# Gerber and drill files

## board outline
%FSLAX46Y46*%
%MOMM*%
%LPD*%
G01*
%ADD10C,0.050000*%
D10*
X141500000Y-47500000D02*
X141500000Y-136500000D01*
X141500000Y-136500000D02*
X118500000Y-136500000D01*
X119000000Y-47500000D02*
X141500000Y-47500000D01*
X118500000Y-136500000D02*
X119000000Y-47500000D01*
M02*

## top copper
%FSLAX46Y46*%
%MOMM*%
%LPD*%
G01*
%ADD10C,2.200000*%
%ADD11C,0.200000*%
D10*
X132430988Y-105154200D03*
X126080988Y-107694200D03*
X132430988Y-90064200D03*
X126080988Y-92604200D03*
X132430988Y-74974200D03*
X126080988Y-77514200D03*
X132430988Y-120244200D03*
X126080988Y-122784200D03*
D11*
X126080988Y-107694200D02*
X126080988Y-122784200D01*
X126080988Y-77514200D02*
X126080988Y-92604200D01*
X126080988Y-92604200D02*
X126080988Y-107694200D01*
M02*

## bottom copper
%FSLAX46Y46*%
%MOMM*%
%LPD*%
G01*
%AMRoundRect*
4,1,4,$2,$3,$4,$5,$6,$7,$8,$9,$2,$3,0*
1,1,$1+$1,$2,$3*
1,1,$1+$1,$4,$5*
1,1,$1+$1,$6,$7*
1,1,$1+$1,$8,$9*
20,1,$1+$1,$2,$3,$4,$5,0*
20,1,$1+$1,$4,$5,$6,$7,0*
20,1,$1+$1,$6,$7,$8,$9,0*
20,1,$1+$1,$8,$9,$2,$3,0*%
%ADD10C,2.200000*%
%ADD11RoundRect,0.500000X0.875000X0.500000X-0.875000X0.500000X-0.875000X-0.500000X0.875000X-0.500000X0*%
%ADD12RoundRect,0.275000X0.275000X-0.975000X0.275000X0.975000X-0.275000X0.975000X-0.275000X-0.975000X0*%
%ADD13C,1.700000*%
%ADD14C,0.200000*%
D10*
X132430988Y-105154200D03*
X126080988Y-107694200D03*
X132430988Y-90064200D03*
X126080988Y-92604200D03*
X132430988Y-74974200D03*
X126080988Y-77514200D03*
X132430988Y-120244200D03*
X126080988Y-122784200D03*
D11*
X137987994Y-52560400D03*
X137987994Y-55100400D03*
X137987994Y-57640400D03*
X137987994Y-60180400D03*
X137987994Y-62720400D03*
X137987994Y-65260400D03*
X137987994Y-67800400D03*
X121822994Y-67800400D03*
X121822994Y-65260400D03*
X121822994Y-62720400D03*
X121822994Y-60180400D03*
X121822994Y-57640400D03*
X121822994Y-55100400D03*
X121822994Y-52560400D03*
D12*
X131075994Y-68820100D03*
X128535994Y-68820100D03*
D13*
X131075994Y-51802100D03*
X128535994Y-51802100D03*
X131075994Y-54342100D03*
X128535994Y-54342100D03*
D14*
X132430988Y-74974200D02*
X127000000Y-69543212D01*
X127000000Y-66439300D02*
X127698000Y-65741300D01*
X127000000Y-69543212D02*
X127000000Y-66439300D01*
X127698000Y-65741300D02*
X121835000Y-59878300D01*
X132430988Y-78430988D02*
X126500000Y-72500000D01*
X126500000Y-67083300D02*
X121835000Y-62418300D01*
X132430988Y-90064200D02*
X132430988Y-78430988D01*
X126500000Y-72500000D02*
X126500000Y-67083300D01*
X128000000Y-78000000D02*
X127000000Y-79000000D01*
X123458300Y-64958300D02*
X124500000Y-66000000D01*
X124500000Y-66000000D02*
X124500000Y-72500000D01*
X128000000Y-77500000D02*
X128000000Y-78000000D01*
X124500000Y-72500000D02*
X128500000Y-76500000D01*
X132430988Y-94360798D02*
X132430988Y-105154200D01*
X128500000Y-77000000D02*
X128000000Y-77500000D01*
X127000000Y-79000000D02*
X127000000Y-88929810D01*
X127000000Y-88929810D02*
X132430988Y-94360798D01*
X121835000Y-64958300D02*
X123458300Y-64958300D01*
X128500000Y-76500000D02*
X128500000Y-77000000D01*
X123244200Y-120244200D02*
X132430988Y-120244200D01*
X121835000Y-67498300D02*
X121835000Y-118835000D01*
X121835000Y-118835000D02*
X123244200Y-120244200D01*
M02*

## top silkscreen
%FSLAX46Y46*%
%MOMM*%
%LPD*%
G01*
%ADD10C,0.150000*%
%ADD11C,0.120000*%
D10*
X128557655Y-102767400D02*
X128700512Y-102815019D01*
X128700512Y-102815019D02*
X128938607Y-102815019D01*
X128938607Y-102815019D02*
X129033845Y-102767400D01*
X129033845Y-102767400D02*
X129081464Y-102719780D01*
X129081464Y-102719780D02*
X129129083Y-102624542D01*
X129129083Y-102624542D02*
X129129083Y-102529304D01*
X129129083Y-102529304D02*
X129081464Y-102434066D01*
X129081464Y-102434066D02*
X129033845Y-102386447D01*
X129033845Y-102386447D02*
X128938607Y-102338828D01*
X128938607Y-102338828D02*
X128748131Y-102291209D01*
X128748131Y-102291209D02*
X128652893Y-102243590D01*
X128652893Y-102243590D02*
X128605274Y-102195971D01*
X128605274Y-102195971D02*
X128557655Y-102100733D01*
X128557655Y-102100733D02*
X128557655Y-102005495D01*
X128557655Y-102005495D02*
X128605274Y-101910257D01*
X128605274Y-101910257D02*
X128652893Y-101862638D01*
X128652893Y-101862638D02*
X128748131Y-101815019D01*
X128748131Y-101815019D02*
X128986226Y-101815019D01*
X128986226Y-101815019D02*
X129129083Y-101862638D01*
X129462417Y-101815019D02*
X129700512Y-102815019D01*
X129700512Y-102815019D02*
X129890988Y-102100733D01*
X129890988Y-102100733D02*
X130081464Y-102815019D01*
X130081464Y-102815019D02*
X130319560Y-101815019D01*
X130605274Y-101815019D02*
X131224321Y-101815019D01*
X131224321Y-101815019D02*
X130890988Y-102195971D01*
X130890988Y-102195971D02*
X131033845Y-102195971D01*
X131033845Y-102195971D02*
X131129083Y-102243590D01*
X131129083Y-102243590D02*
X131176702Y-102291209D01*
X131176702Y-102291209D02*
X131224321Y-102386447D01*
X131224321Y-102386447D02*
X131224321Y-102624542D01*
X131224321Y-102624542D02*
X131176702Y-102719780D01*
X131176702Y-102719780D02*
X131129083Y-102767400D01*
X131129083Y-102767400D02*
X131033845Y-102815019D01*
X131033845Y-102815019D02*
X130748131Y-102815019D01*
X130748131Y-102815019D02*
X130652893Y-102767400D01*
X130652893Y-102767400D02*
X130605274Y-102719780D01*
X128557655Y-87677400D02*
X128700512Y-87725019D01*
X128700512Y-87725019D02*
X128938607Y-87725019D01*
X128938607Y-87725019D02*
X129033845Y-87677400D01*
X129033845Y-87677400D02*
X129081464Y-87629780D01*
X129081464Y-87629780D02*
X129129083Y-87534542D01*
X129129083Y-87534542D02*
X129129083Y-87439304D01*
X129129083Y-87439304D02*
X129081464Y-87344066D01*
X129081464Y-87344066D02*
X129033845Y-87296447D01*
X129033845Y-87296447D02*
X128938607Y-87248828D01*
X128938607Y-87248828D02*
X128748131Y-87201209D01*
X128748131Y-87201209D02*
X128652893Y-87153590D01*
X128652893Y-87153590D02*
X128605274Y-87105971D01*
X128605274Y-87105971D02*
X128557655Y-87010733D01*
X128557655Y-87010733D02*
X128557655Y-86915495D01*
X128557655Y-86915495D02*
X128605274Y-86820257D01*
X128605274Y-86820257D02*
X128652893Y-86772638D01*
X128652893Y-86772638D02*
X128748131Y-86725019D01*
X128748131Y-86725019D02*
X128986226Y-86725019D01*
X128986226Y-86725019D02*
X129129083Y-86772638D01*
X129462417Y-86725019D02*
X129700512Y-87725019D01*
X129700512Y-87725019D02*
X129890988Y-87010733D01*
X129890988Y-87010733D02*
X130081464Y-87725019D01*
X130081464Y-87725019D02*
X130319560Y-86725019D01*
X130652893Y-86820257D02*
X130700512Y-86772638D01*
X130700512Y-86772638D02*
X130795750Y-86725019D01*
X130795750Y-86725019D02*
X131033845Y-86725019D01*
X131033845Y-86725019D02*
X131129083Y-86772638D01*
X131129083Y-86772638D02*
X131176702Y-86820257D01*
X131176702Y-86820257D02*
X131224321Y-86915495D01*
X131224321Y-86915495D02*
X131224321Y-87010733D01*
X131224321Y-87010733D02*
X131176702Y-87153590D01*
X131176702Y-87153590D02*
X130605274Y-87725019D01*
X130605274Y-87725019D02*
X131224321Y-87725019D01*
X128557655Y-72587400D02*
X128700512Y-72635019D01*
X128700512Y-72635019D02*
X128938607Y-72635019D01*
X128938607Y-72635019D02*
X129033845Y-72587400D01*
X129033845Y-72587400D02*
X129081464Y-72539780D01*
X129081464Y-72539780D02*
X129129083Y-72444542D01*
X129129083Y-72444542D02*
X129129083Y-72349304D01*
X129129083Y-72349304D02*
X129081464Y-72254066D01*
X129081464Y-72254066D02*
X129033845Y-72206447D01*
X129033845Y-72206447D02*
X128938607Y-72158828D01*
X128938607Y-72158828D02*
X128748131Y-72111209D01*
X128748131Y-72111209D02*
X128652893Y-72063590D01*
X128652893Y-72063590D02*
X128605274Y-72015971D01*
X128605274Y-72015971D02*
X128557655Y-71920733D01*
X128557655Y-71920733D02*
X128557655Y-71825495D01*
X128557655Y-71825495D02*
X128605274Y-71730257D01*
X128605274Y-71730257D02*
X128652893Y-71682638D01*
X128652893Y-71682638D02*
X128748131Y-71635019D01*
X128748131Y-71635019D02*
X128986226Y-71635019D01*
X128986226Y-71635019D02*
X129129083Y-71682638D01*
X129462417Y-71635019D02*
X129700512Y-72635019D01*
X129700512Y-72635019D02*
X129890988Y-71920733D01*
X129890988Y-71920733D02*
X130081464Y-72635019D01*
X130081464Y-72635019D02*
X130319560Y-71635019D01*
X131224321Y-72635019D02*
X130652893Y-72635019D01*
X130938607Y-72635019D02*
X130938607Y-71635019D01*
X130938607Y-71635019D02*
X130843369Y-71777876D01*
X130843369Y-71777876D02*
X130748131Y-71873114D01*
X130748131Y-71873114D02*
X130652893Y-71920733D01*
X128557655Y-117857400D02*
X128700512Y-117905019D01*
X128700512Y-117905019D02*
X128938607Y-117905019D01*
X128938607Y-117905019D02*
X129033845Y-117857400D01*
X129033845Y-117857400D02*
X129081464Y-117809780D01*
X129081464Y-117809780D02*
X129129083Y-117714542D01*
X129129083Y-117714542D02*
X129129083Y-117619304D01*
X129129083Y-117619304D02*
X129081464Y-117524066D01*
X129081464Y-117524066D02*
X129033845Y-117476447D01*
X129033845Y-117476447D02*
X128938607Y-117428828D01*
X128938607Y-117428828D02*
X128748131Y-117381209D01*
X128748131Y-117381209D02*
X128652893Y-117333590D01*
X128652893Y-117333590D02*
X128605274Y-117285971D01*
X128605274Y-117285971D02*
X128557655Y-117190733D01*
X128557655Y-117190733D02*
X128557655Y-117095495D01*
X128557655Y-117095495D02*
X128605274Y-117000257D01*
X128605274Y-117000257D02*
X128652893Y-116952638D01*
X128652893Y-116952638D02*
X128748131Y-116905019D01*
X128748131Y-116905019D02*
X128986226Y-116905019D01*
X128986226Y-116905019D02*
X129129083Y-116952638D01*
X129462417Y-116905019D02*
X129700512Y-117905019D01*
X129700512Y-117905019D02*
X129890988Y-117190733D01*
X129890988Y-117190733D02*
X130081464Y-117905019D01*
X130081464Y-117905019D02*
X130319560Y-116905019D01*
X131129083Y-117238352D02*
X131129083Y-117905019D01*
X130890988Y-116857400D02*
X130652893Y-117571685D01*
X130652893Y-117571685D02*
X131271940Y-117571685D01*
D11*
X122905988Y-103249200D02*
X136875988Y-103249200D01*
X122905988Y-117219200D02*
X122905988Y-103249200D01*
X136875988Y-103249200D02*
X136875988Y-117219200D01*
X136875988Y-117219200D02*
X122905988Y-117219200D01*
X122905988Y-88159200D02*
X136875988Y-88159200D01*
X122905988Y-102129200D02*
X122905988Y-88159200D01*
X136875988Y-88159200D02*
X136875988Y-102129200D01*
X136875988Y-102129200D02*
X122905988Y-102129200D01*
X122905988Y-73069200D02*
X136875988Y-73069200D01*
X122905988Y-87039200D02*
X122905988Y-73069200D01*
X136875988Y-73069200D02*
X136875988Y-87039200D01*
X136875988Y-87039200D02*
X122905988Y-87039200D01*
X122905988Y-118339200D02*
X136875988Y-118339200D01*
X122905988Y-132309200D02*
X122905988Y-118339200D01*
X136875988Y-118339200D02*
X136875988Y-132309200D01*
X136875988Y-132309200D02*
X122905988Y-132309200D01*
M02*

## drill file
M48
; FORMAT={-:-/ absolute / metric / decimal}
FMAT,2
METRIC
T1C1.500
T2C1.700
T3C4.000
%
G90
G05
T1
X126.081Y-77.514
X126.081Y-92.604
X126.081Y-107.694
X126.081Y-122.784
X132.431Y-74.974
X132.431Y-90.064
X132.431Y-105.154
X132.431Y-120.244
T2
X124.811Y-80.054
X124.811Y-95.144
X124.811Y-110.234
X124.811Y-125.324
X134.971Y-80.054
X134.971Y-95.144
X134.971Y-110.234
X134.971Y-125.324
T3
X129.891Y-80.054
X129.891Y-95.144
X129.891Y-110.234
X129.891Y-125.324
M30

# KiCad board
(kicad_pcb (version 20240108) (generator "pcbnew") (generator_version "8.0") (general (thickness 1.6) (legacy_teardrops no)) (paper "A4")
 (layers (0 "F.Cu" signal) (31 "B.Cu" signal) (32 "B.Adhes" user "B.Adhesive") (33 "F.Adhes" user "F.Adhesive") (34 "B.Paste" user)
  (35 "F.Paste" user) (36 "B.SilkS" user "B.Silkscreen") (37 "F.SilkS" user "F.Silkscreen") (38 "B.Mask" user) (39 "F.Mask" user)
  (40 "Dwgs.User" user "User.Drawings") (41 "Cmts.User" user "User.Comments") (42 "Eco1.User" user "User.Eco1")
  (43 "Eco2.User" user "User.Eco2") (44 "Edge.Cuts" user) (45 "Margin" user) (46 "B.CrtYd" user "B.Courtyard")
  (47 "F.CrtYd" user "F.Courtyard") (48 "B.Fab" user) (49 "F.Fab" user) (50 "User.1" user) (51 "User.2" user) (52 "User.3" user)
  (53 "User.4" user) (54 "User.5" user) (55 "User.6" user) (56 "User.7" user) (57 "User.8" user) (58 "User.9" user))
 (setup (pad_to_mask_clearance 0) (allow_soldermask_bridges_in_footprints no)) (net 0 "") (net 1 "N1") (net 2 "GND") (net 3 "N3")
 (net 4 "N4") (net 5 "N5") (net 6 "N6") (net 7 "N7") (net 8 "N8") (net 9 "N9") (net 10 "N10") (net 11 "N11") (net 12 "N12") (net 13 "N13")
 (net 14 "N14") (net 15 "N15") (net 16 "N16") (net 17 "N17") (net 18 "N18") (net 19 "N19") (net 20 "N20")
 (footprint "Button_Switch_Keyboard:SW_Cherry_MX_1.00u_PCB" (layer "F.Cu") (at 132.430988 105.1542)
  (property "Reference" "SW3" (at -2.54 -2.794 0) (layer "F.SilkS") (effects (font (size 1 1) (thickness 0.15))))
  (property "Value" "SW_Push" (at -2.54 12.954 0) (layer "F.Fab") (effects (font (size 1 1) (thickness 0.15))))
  (fp_line (start -9.525 -1.905) (end 4.445 -1.905) (stroke (width 0.12) (type solid)) (layer "F.SilkS"))
  (fp_line (start -9.525 12.065) (end -9.525 -1.905) (stroke (width 0.12) (type solid)) (layer "F.SilkS"))
  (fp_line (start 4.445 -1.905) (end 4.445 12.065) (stroke (width 0.12) (type solid)) (layer "F.SilkS"))
  (fp_line (start 4.445 12.065) (end -9.525 12.065) (stroke (width 0.12) (type solid)) (layer "F.SilkS"))
  (pad "" np_thru_hole circle (at -7.62 5.08) (size 1.7 1.7) (drill 1.7) (layers "*.Cu" "*.Mask"))
  (pad "" np_thru_hole circle (at -2.54 5.08) (size 4 4) (drill 4) (layers "*.Cu" "*.Mask"))
  (pad "" np_thru_hole circle (at 2.54 5.08) (size 1.7 1.7) (drill 1.7) (layers "*.Cu" "*.Mask"))
  (pad "1" thru_hole circle (at 0 0) (size 2.2 2.2) (drill 1.5) (layers "*.Cu" "*.Mask") (remove_unused_layers no) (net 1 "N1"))
  (pad "2" thru_hole circle (at -6.35 2.54) (size 2.2 2.2) (drill 1.5) (layers "*.Cu" "*.Mask") (remove_unused_layers no) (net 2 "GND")))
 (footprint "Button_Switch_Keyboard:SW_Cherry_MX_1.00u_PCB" (layer "F.Cu") (at 132.430988 90.0642)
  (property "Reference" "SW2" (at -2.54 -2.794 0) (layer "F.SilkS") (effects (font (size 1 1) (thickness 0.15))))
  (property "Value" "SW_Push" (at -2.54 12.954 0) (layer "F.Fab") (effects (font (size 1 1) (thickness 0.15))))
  (fp_line (start -9.525 -1.905) (end 4.445 -1.905) (stroke (width 0.12) (type solid)) (layer "F.SilkS"))
  (fp_line (start -9.525 12.065) (end -9.525 -1.905) (stroke (width 0.12) (type solid)) (layer "F.SilkS"))
  (fp_line (start 4.445 -1.905) (end 4.445 12.065) (stroke (width 0.12) (type solid)) (layer "F.SilkS"))
  (fp_line (start 4.445 12.065) (end -9.525 12.065) (stroke (width 0.12) (type solid)) (layer "F.SilkS"))
  (pad "" np_thru_hole circle (at -7.62 5.08) (size 1.7 1.7) (drill 1.7) (layers "*.Cu" "*.Mask"))
  (pad "" np_thru_hole circle (at -2.54 5.08) (size 4 4) (drill 4) (layers "*.Cu" "*.Mask"))
  (pad "" np_thru_hole circle (at 2.54 5.08) (size 1.7 1.7) (drill 1.7) (layers "*.Cu" "*.Mask"))
  (pad "1" thru_hole circle (at 0 0) (size 2.2 2.2) (drill 1.5) (layers "*.Cu" "*.Mask") (remove_unused_layers no) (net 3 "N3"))
  (pad "2" thru_hole circle (at -6.35 2.54) (size 2.2 2.2) (drill 1.5) (layers "*.Cu" "*.Mask") (remove_unused_layers no) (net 2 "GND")))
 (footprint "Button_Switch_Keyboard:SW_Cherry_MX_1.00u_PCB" (layer "F.Cu") (at 132.430988 74.9742)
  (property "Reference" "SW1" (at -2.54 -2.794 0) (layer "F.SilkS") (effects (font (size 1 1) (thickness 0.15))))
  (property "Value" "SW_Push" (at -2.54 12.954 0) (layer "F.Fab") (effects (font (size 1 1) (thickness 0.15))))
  (fp_line (start -9.525 -1.905) (end 4.445 -1.905) (stroke (width 0.12) (type solid)) (layer "F.SilkS"))
  (fp_line (start -9.525 12.065) (end -9.525 -1.905) (stroke (width 0.12) (type solid)) (layer "F.SilkS"))
  (fp_line (start 4.445 -1.905) (end 4.445 12.065) (stroke (width 0.12) (type solid)) (layer "F.SilkS"))
  (fp_line (start 4.445 12.065) (end -9.525 12.065) (stroke (width 0.12) (type solid)) (layer "F.SilkS"))
  (pad "" np_thru_hole circle (at -7.62 5.08) (size 1.7 1.7) (drill 1.7) (layers "*.Cu" "*.Mask"))
  (pad "" np_thru_hole circle (at -2.54 5.08) (size 4 4) (drill 4) (layers "*.Cu" "*.Mask"))
  (pad "" np_thru_hole circle (at 2.54 5.08) (size 1.7 1.7) (drill 1.7) (layers "*.Cu" "*.Mask"))
  (pad "1" thru_hole circle (at 0 0) (size 2.2 2.2) (drill 1.5) (layers "*.Cu" "*.Mask") (remove_unused_layers no) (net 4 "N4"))
  (pad "2" thru_hole circle (at -6.35 2.54) (size 2.2 2.2) (drill 1.5) (layers "*.Cu" "*.Mask") (remove_unused_layers no) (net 2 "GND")))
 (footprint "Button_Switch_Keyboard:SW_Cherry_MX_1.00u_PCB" (layer "F.Cu") (at 132.430988 120.2442)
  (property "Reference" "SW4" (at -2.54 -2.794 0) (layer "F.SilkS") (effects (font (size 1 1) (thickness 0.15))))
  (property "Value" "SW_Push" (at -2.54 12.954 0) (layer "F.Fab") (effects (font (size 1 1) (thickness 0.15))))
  (fp_line (start -9.525 -1.905) (end 4.445 -1.905) (stroke (width 0.12) (type solid)) (layer "F.SilkS"))
  (fp_line (start -9.525 12.065) (end -9.525 -1.905) (stroke (width 0.12) (type solid)) (layer "F.SilkS"))
  (fp_line (start 4.445 -1.905) (end 4.445 12.065) (stroke (width 0.12) (type solid)) (layer "F.SilkS"))
  (fp_line (start 4.445 12.065) (end -9.525 12.065) (stroke (width 0.12) (type solid)) (layer "F.SilkS"))
  (pad "" np_thru_hole circle (at -7.62 5.08) (size 1.7 1.7) (drill 1.7) (layers "*.Cu" "*.Mask"))
  (pad "" np_thru_hole circle (at -2.54 5.08) (size 4 4) (drill 4) (layers "*.Cu" "*.Mask"))
  (pad "" np_thru_hole circle (at 2.54 5.08) (size 1.7 1.7) (drill 1.7) (layers "*.Cu" "*.Mask"))
  (pad "1" thru_hole circle (at 0 0) (size 2.2 2.2) (drill 1.5) (layers "*.Cu" "*.Mask") (remove_unused_layers no) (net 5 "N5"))
  (pad "2" thru_hole circle (at -6.35 2.54) (size 2.2 2.2) (drill 1.5) (layers "*.Cu" "*.Mask") (remove_unused_layers no) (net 2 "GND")))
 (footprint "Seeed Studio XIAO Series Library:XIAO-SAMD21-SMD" (layer "B.Cu") (at 138.822994 70.6804 180)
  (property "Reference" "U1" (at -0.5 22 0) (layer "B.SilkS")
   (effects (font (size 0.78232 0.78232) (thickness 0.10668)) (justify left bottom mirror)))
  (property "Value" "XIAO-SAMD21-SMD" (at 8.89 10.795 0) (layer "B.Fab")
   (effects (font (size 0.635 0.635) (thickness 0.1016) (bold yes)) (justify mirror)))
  (pad "1" smd roundrect (at 0.835 18.12 180) (size 2.75 2) (layers "B.Cu" "B.Paste" "B.Mask") (roundrect_rratio 0.25) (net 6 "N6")
   (solder_mask_margin 0.0508) (thermal_bridge_angle 45))
  (pad "2" smd roundrect (at 0.835 15.58 180) (size 2.75 2) (layers "B.Cu" "B.Paste" "B.Mask") (roundrect_rratio 0.25) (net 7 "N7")
   (solder_mask_margin 0.0508) (thermal_bridge_angle 45))
  (pad "3" smd roundrect (at 0.835 13.04 180) (size 2.75 2) (layers "B.Cu" "B.Paste" "B.Mask") (roundrect_rratio 0.25) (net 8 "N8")
   (solder_mask_margin 0.0508) (thermal_bridge_angle 45))
  (pad "4" smd roundrect (at 0.835 10.5 180) (size 2.75 2) (layers "B.Cu" "B.Paste" "B.Mask") (roundrect_rratio 0.25) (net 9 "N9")
   (solder_mask_margin 0.0508) (thermal_bridge_angle 45))
  (pad "5" smd roundrect (at 0.835 7.96 180) (size 2.75 2) (layers "B.Cu" "B.Paste" "B.Mask") (roundrect_rratio 0.25) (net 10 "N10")
   (solder_mask_margin 0.0508) (thermal_bridge_angle 45))
  (pad "6" smd roundrect (at 0.835 5.42 180) (size 2.75 2) (layers "B.Cu" "B.Paste" "B.Mask") (roundrect_rratio 0.25) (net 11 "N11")
   (solder_mask_margin 0.0508) (thermal_bridge_angle 45))
  (pad "7" smd roundrect (at 0.835 2.88 180) (size 2.75 2) (layers "B.Cu" "B.Paste" "B.Mask") (roundrect_rratio 0.25) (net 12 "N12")
   (solder_mask_margin 0.0508) (thermal_bridge_angle 45))
  (pad "8" smd roundrect (at 17 2.88 180) (size 2.75 2) (layers "B.Cu" "B.Paste" "B.Mask") (roundrect_rratio 0.25) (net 5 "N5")
   (solder_mask_margin 0.0508) (thermal_bridge_angle 45))
  (pad "9" smd roundrect (at 17 5.42 180) (size 2.75 2) (layers "B.Cu" "B.Paste" "B.Mask") (roundrect_rratio 0.25) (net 1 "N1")
   (solder_mask_margin 0.0508) (thermal_bridge_angle 45))
  (pad "10" smd roundrect (at 17 7.96 180) (size 2.75 2) (layers "B.Cu" "B.Paste" "B.Mask") (roundrect_rratio 0.25) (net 3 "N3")
   (solder_mask_margin 0.0508) (thermal_bridge_angle 45))
  (pad "11" smd roundrect (at 17 10.5 180) (size 2.75 2) (layers "B.Cu" "B.Paste" "B.Mask") (roundrect_rratio 0.25) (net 4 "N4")
   (solder_mask_margin 0.0508) (thermal_bridge_angle 45))
  (pad "12" smd roundrect (at 17 13.04 180) (size 2.75 2) (layers "B.Cu" "B.Paste" "B.Mask") (roundrect_rratio 0.25) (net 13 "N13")
   (solder_mask_margin 0.0508) (thermal_bridge_angle 45))
  (pad "13" smd roundrect (at 17 15.58 180) (size 2.75 2) (layers "B.Cu" "B.Paste" "B.Mask") (roundrect_rratio 0.25) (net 2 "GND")
   (solder_mask_margin 0.0508) (thermal_bridge_angle 45))
  (pad "14" smd roundrect (at 17 18.12 180) (size 2.75 2) (layers "B.Cu" "B.Paste" "B.Mask") (roundrect_rratio 0.25) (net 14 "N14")
   (solder_mask_margin 0.0508) (thermal_bridge_angle 45))
  (pad "15" smd roundrect (at 7.747 1.8603 90) (size 2.5 1.1) (layers "B.Cu" "B.Paste" "B.Mask") (roundrect_rratio 0.25) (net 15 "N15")
   (solder_mask_margin 0.0508) (thermal_bridge_angle 45))
  (pad "16" smd roundrect (at 10.287 1.8603 90) (size 2.5 1.1) (layers "B.Cu" "B.Paste" "B.Mask") (roundrect_rratio 0.25) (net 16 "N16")
   (solder_mask_margin 0.0508) (thermal_bridge_angle 45))
  (pad "17" smd circle (at 7.747 18.8783 180) (size 1.7 1.7) (layers "B.Cu" "B.Paste" "B.Mask") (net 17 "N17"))
  (pad "18" smd circle (at 10.287 18.8783 180) (size 1.7 1.7) (layers "B.Cu" "B.Paste" "B.Mask") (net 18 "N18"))
  (pad "19" smd circle (at 7.747 16.3383 180) (size 1.7 1.7) (layers "B.Cu" "B.Paste" "B.Mask") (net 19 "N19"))
  (pad "20" smd circle (at 10.287 16.3383 180) (size 1.7 1.7) (layers "B.Cu" "B.Paste" "B.Mask") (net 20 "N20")))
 (gr_line (start 141.5 47.5) (end 141.5 136.5) (stroke (width 0.05) (type default)) (layer "Edge.Cuts"))
 (gr_line (start 141.5 136.5) (end 118.5 136.5) (stroke (width 0.05) (type default)) (layer "Edge.Cuts"))
 (gr_line (start 119 47.5) (end 141.5 47.5) (stroke (width 0.05) (type default)) (layer "Edge.Cuts"))
 (gr_line (start 118.5 136.5) (end 119 47.5) (stroke (width 0.05) (type default)) (layer "Edge.Cuts"))
 (segment (start 126.080988 107.6942) (end 126.080988 122.7842) (width 0.2) (layer "F.Cu") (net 2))
 (segment (start 126.080988 77.5142) (end 126.080988 92.6042) (width 0.2) (layer "F.Cu") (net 2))
 (segment (start 126.080988 92.6042) (end 126.080988 107.6942) (width 0.2) (layer "F.Cu") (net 2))
 (segment (start 132.430988 74.9742) (end 127 69.543212) (width 0.2) (layer "B.Cu") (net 4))
 (segment (start 127 66.4393) (end 127.698 65.7413) (width 0.2) (layer "B.Cu") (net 4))
 (segment (start 127 69.543212) (end 127 66.4393) (width 0.2) (layer "B.Cu") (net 4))
 (segment (start 127.698 65.7413) (end 121.835 59.8783) (width 0.2) (layer "B.Cu") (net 4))
 (segment (start 132.430988 78.430988) (end 126.5 72.5) (width 0.2) (layer "B.Cu") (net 3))
 (segment (start 126.5 67.0833) (end 121.835 62.4183) (width 0.2) (layer "B.Cu") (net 3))
 (segment (start 132.430988 90.0642) (end 132.430988 78.430988) (width 0.2) (layer "B.Cu") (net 3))
 (segment (start 126.5 72.5) (end 126.5 67.0833) (width 0.2) (layer "B.Cu") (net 3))
 (segment (start 128 78) (end 127 79) (width 0.2) (layer "B.Cu") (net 1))
 (segment (start 123.4583 64.9583) (end 124.5 66) (width 0.2) (layer "B.Cu") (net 1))
 (segment (start 124.5 66) (end 124.5 72.5) (width 0.2) (layer "B.Cu") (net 1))
 (segment (start 128 77.5) (end 128 78) (width 0.2) (layer "B.Cu") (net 1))
 (segment (start 124.5 72.5) (end 128.5 76.5) (width 0.2) (layer "B.Cu") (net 1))
 (segment (start 132.430988 94.360798) (end 132.430988 105.1542) (width 0.2) (layer "B.Cu") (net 1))
 (segment (start 128.5 77) (end 128 77.5) (width 0.2) (layer "B.Cu") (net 1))
 (segment (start 127 79) (end 127 88.92981) (width 0.2) (layer "B.Cu") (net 1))
 (segment (start 127 88.92981) (end 132.430988 94.360798) (width 0.2) (layer "B.Cu") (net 1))
 (segment (start 121.835 64.9583) (end 123.4583 64.9583) (width 0.2) (layer "B.Cu") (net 1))
 (segment (start 128.5 76.5) (end 128.5 77) (width 0.2) (layer "B.Cu") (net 1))
 (segment (start 123.2442 120.2442) (end 132.430988 120.2442) (width 0.2) (layer "B.Cu") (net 5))
 (segment (start 121.835 67.4983) (end 121.835 118.835) (width 0.2) (layer "B.Cu") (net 5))
 (segment (start 121.835 118.835) (end 123.2442 120.2442) (width 0.2) (layer "B.Cu") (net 5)))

